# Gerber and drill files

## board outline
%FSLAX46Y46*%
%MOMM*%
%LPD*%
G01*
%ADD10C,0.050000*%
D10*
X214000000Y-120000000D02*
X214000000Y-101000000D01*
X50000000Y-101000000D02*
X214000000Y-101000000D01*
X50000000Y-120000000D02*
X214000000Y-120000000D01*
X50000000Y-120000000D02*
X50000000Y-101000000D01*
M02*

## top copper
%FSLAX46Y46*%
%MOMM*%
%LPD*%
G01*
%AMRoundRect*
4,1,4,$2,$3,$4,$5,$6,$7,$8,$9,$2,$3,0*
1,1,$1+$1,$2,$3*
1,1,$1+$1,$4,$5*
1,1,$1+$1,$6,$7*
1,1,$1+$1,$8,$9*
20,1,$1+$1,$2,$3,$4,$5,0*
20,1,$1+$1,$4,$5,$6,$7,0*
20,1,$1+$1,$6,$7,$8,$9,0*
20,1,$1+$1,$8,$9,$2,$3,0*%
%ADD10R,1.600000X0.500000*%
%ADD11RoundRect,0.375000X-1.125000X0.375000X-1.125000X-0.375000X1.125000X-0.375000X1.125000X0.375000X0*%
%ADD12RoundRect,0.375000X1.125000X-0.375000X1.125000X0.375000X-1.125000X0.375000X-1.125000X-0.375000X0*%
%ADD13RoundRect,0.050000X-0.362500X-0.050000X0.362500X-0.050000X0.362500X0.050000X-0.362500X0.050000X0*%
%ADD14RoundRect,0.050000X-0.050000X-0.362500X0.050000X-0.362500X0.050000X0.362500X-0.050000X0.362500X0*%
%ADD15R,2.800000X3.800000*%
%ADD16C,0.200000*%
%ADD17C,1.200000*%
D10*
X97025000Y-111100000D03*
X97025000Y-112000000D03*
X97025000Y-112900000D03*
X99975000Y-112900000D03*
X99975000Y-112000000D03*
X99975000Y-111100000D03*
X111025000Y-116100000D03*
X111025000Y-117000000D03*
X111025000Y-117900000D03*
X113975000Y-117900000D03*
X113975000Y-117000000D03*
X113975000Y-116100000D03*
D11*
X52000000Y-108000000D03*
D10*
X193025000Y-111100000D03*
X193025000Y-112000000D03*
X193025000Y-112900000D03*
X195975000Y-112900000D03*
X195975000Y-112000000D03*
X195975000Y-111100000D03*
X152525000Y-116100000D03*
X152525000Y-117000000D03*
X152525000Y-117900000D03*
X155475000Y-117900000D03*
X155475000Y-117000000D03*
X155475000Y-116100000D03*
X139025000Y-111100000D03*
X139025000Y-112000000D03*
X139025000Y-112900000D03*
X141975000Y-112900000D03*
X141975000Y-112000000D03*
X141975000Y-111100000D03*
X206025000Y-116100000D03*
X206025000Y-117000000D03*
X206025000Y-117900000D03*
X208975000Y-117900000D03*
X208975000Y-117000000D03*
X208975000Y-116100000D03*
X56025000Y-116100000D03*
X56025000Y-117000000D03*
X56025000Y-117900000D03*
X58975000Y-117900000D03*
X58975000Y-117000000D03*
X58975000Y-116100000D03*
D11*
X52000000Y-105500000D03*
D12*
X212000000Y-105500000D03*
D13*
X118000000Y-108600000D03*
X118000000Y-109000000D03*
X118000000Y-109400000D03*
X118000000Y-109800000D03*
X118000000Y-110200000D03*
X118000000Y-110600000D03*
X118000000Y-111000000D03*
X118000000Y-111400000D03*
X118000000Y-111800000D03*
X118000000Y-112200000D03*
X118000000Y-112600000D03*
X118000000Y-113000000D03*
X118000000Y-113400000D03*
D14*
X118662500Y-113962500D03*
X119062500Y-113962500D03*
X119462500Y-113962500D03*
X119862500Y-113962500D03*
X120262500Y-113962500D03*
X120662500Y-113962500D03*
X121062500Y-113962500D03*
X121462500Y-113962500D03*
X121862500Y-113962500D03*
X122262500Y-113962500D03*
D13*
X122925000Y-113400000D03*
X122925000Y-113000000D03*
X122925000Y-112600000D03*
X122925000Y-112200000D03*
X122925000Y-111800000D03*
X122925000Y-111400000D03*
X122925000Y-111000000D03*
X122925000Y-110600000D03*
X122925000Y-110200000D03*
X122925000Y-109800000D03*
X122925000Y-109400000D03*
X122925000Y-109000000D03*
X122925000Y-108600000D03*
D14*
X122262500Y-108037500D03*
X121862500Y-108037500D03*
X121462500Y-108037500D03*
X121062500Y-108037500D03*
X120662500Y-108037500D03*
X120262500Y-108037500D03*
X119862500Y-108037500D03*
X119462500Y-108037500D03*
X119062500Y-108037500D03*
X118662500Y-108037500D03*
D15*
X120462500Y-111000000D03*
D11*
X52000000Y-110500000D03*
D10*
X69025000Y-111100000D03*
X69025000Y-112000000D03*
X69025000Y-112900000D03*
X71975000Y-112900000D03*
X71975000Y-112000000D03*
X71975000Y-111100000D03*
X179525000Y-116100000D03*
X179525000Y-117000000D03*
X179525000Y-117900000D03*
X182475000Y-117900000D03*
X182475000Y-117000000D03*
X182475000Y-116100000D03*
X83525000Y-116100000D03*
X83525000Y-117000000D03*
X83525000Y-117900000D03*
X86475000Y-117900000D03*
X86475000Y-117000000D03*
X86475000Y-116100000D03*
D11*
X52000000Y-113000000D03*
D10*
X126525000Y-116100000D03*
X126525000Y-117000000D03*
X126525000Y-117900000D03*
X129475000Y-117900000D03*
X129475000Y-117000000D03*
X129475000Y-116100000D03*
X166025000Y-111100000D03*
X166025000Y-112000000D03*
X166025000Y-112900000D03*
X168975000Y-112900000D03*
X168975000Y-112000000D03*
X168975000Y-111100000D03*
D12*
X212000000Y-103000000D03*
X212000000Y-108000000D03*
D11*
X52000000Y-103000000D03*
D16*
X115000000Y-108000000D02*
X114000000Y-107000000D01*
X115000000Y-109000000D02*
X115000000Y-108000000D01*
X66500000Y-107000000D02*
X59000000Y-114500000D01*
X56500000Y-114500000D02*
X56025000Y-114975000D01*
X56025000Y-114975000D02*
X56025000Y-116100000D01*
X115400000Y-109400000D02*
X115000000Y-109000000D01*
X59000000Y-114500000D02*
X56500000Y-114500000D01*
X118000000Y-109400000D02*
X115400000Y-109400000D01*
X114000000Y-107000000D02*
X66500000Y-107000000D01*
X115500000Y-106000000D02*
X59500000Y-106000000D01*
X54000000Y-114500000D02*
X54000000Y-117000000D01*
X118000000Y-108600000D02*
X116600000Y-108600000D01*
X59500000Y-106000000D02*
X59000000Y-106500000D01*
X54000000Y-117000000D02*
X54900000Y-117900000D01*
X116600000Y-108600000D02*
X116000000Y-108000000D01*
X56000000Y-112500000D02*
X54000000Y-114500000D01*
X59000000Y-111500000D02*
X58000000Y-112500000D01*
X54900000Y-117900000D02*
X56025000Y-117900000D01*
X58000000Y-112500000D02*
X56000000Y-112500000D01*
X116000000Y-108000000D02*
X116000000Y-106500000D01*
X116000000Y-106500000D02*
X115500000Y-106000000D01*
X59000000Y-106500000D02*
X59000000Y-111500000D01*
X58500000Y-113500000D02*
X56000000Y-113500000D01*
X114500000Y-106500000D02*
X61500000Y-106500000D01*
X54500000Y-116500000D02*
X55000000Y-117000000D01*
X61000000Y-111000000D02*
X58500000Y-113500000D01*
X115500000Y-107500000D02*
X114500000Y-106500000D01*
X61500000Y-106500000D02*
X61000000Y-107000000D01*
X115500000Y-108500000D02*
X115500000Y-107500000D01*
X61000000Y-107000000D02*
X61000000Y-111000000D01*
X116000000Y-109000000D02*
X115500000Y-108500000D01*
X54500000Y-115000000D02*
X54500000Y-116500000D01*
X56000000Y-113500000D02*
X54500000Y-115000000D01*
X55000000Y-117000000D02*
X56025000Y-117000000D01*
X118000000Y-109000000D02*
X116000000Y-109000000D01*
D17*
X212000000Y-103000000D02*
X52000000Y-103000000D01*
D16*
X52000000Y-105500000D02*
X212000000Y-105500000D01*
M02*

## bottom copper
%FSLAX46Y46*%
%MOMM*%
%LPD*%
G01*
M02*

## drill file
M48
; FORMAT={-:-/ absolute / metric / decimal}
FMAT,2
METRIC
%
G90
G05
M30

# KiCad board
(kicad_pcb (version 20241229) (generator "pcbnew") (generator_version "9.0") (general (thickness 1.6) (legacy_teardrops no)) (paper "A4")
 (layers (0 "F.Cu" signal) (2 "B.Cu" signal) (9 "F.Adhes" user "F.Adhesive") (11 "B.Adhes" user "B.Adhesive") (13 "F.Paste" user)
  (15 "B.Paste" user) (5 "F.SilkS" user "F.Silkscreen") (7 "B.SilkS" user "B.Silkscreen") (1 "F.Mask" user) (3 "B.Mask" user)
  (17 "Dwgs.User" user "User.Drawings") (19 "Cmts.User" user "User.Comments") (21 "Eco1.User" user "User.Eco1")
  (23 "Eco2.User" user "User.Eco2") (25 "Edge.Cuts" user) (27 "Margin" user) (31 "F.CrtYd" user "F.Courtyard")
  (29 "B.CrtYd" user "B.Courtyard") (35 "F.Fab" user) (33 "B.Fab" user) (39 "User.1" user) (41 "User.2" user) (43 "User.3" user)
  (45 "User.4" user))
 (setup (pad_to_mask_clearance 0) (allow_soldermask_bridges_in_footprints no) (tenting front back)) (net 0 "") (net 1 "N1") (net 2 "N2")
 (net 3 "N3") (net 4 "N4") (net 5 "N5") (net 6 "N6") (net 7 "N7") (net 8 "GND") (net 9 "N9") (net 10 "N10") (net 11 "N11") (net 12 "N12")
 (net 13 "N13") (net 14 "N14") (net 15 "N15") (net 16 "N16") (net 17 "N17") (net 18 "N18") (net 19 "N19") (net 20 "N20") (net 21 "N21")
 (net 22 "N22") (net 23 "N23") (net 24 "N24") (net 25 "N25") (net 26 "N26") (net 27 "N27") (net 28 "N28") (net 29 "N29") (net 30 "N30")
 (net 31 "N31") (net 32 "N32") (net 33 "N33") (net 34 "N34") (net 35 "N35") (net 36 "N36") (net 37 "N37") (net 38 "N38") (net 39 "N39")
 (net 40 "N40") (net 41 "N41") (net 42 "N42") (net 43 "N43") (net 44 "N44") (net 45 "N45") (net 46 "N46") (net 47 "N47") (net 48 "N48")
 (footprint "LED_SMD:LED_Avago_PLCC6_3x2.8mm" (layer "F.Cu") (at 98.5 112)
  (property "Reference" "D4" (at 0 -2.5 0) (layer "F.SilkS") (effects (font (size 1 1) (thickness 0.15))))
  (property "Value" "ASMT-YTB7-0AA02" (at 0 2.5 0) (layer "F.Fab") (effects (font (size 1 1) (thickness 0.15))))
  (pad "1" smd rect (at -1.475 -0.9) (size 1.6 0.5) (layers "F.Cu" "F.Mask" "F.Paste") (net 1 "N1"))
  (pad "2" smd rect (at -1.475 0) (size 1.6 0.5) (layers "F.Cu" "F.Mask" "F.Paste") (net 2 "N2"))
  (pad "3" smd rect (at -1.475 0.9) (size 1.6 0.5) (layers "F.Cu" "F.Mask" "F.Paste") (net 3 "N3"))
  (pad "4" smd rect (at 1.475 0.9) (size 1.6 0.5) (layers "F.Cu" "F.Mask" "F.Paste") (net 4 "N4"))
  (pad "5" smd rect (at 1.475 0) (size 1.6 0.5) (layers "F.Cu" "F.Mask" "F.Paste") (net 4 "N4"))
  (pad "6" smd rect (at 1.475 -0.9) (size 1.6 0.5) (layers "F.Cu" "F.Mask" "F.Paste") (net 4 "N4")))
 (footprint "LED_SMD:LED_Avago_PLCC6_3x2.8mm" (layer "F.Cu") (at 112.5 117)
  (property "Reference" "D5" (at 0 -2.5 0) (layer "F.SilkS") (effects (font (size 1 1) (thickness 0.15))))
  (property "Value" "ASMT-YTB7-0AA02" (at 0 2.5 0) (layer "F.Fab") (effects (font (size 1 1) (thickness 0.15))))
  (pad "1" smd rect (at -1.475 -0.9) (size 1.6 0.5) (layers "F.Cu" "F.Mask" "F.Paste") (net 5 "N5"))
  (pad "2" smd rect (at -1.475 0) (size 1.6 0.5) (layers "F.Cu" "F.Mask" "F.Paste") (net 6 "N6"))
  (pad "3" smd rect (at -1.475 0.9) (size 1.6 0.5) (layers "F.Cu" "F.Mask" "F.Paste") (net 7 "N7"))
  (pad "4" smd rect (at 1.475 0.9) (size 1.6 0.5) (layers "F.Cu" "F.Mask" "F.Paste") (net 4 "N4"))
  (pad "5" smd rect (at 1.475 0) (size 1.6 0.5) (layers "F.Cu" "F.Mask" "F.Paste") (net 4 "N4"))
  (pad "6" smd rect (at 1.475 -0.9) (size 1.6 0.5) (layers "F.Cu" "F.Mask" "F.Paste") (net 4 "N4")))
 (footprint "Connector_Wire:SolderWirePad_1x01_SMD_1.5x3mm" (layer "F.Cu") (at 52 108 -90)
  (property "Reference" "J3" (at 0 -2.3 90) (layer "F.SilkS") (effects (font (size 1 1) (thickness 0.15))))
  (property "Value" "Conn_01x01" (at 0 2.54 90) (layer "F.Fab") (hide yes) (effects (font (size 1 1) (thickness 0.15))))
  (pad "1" smd roundrect (at 0 0 270) (size 1.5 3) (layers "F.Cu" "F.Mask") (roundrect_rratio 0.25) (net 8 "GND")))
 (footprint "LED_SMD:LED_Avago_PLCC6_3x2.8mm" (layer "F.Cu") (at 194.5 112)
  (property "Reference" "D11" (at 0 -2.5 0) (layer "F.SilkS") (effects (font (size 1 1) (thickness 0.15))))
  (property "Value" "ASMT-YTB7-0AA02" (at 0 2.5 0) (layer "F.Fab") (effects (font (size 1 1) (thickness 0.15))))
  (pad "1" smd rect (at -1.475 -0.9) (size 1.6 0.5) (layers "F.Cu" "F.Mask" "F.Paste") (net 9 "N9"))
  (pad "2" smd rect (at -1.475 0) (size 1.6 0.5) (layers "F.Cu" "F.Mask" "F.Paste") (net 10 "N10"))
  (pad "3" smd rect (at -1.475 0.9) (size 1.6 0.5) (layers "F.Cu" "F.Mask" "F.Paste") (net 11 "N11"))
  (pad "4" smd rect (at 1.475 0.9) (size 1.6 0.5) (layers "F.Cu" "F.Mask" "F.Paste") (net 4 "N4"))
  (pad "5" smd rect (at 1.475 0) (size 1.6 0.5) (layers "F.Cu" "F.Mask" "F.Paste") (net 4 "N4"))
  (pad "6" smd rect (at 1.475 -0.9) (size 1.6 0.5) (layers "F.Cu" "F.Mask" "F.Paste") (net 4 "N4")))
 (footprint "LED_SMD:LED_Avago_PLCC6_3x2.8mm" (layer "F.Cu") (at 154 117)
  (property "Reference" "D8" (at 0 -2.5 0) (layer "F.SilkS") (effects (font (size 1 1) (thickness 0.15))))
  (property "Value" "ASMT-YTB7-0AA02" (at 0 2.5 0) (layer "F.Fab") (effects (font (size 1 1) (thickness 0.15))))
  (pad "1" smd rect (at -1.475 -0.9) (size 1.6 0.5) (layers "F.Cu" "F.Mask" "F.Paste") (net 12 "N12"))
  (pad "2" smd rect (at -1.475 0) (size 1.6 0.5) (layers "F.Cu" "F.Mask" "F.Paste") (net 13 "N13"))
  (pad "3" smd rect (at -1.475 0.9) (size 1.6 0.5) (layers "F.Cu" "F.Mask" "F.Paste") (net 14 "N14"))
  (pad "4" smd rect (at 1.475 0.9) (size 1.6 0.5) (layers "F.Cu" "F.Mask" "F.Paste") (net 4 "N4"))
  (pad "5" smd rect (at 1.475 0) (size 1.6 0.5) (layers "F.Cu" "F.Mask" "F.Paste") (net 4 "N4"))
  (pad "6" smd rect (at 1.475 -0.9) (size 1.6 0.5) (layers "F.Cu" "F.Mask" "F.Paste") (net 4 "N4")))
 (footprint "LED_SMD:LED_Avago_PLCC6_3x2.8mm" (layer "F.Cu") (at 140.5 112)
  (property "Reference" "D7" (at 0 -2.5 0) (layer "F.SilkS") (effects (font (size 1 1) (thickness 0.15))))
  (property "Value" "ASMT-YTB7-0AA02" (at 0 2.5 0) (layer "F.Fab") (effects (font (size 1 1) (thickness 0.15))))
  (pad "1" smd rect (at -1.475 -0.9) (size 1.6 0.5) (layers "F.Cu" "F.Mask" "F.Paste") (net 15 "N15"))
  (pad "2" smd rect (at -1.475 0) (size 1.6 0.5) (layers "F.Cu" "F.Mask" "F.Paste") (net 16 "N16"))
  (pad "3" smd rect (at -1.475 0.9) (size 1.6 0.5) (layers "F.Cu" "F.Mask" "F.Paste") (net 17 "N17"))
  (pad "4" smd rect (at 1.475 0.9) (size 1.6 0.5) (layers "F.Cu" "F.Mask" "F.Paste") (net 4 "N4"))
  (pad "5" smd rect (at 1.475 0) (size 1.6 0.5) (layers "F.Cu" "F.Mask" "F.Paste") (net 4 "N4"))
  (pad "6" smd rect (at 1.475 -0.9) (size 1.6 0.5) (layers "F.Cu" "F.Mask" "F.Paste") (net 4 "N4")))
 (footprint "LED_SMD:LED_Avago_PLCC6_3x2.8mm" (layer "F.Cu") (at 207.5 117)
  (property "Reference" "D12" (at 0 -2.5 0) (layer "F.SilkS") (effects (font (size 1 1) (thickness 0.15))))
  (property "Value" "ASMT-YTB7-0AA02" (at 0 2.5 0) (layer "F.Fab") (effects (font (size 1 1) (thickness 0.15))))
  (pad "1" smd rect (at -1.475 -0.9) (size 1.6 0.5) (layers "F.Cu" "F.Mask" "F.Paste") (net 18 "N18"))
  (pad "2" smd rect (at -1.475 0) (size 1.6 0.5) (layers "F.Cu" "F.Mask" "F.Paste") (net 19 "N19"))
  (pad "3" smd rect (at -1.475 0.9) (size 1.6 0.5) (layers "F.Cu" "F.Mask" "F.Paste") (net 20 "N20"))
  (pad "4" smd rect (at 1.475 0.9) (size 1.6 0.5) (layers "F.Cu" "F.Mask" "F.Paste") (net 4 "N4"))
  (pad "5" smd rect (at 1.475 0) (size 1.6 0.5) (layers "F.Cu" "F.Mask" "F.Paste") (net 4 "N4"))
  (pad "6" smd rect (at 1.475 -0.9) (size 1.6 0.5) (layers "F.Cu" "F.Mask" "F.Paste") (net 4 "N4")))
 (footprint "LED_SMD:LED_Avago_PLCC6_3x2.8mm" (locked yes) (layer "F.Cu") (at 57.5 117)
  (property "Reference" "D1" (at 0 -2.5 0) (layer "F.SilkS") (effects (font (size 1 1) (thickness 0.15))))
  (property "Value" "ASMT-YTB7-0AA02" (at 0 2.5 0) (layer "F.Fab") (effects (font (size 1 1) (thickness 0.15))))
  (pad "1" smd rect (at -1.475 -0.9) (size 1.6 0.5) (layers "F.Cu" "F.Mask" "F.Paste") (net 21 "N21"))
  (pad "2" smd rect (at -1.475 0) (size 1.6 0.5) (layers "F.Cu" "F.Mask" "F.Paste") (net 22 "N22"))
  (pad "3" smd rect (at -1.475 0.9) (size 1.6 0.5) (layers "F.Cu" "F.Mask" "F.Paste") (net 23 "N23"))
  (pad "4" smd rect (at 1.475 0.9) (size 1.6 0.5) (layers "F.Cu" "F.Mask" "F.Paste") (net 4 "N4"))
  (pad "5" smd rect (at 1.475 0) (size 1.6 0.5) (layers "F.Cu" "F.Mask" "F.Paste") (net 4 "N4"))
  (pad "6" smd rect (at 1.475 -0.9) (size 1.6 0.5) (layers "F.Cu" "F.Mask" "F.Paste") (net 4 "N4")))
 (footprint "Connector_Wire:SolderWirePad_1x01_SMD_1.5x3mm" (layer "F.Cu") (at 52 105.5 -90)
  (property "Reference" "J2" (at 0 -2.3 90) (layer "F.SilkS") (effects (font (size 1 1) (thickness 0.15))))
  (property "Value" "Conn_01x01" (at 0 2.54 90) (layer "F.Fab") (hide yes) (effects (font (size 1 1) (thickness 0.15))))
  (pad "1" smd roundrect (at 0 0 270) (size 1.5 3) (layers "F.Cu" "F.Mask") (roundrect_rratio 0.25) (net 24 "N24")))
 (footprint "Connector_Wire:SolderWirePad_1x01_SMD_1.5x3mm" (layer "F.Cu") (at 212 105.5 90)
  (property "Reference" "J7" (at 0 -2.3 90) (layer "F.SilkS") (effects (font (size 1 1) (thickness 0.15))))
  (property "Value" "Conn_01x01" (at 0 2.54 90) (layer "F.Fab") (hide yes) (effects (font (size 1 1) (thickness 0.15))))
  (pad "1" smd roundrect (at 0 0 90) (size 1.5 3) (layers "F.Cu" "F.Mask") (roundrect_rratio 0.25) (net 24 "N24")))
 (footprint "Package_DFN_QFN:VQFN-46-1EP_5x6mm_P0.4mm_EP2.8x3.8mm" (layer "F.Cu") (at 120.4625 111)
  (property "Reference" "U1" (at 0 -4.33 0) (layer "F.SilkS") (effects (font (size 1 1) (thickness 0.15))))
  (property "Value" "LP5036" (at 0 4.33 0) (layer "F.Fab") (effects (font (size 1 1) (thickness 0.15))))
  (pad "" smd roundrect (at -0.7 -1.27) (size 1.13 1.02) (layers "F.Paste") (roundrect_rratio 0.245098))
  (pad "" smd roundrect (at -0.7 0) (size 1.13 1.02) (layers "F.Paste") (roundrect_rratio 0.245098))
  (pad "" smd roundrect (at -0.7 1.27) (size 1.13 1.02) (layers "F.Paste") (roundrect_rratio 0.245098))
  (pad "" smd roundrect (at 0.7 -1.27) (size 1.13 1.02) (layers "F.Paste") (roundrect_rratio 0.245098))
  (pad "" smd roundrect (at 0.7 0) (size 1.13 1.02) (layers "F.Paste") (roundrect_rratio 0.245098))
  (pad "" smd roundrect (at 0.7 1.27) (size 1.13 1.02) (layers "F.Paste") (roundrect_rratio 0.245098))
  (pad "1" smd roundrect (at -2.4625 -2.4) (size 0.825 0.2) (layers "F.Cu" "F.Mask" "F.Paste") (roundrect_rratio 0.25) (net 23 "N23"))
  (pad "2" smd roundrect (at -2.4625 -2) (size 0.825 0.2) (layers "F.Cu" "F.Mask" "F.Paste") (roundrect_rratio 0.25) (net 22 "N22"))
  (pad "3" smd roundrect (at -2.4625 -1.6) (size 0.825 0.2) (layers "F.Cu" "F.Mask" "F.Paste") (roundrect_rratio 0.25) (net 21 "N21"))
  (pad "4" smd roundrect (at -2.4625 -1.2) (size 0.825 0.2) (layers "F.Cu" "F.Mask" "F.Paste") (roundrect_rratio 0.25) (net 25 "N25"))
  (pad "5" smd roundrect (at -2.4625 -0.8) (size 0.825 0.2) (layers "F.Cu" "F.Mask" "F.Paste") (roundrect_rratio 0.25) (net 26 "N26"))
  (pad "6" smd roundrect (at -2.4625 -0.4) (size 0.825 0.2) (layers "F.Cu" "F.Mask" "F.Paste") (roundrect_rratio 0.25) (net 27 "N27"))
  (pad "7" smd roundrect (at -2.4625 0) (size 0.825 0.2) (layers "F.Cu" "F.Mask" "F.Paste") (roundrect_rratio 0.25) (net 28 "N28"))
  (pad "8" smd roundrect (at -2.4625 0.4) (size 0.825 0.2) (layers "F.Cu" "F.Mask" "F.Paste") (roundrect_rratio 0.25) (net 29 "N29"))
  (pad "9" smd roundrect (at -2.4625 0.8) (size 0.825 0.2) (layers "F.Cu" "F.Mask" "F.Paste") (roundrect_rratio 0.25) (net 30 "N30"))
  (pad "10" smd roundrect (at -2.4625 1.2) (size 0.825 0.2) (layers "F.Cu" "F.Mask" "F.Paste") (roundrect_rratio 0.25) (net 3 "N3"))
  (pad "11" smd roundrect (at -2.4625 1.6) (size 0.825 0.2) (layers "F.Cu" "F.Mask" "F.Paste") (roundrect_rratio 0.25) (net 2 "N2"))
  (pad "12" smd roundrect (at -2.4625 2) (size 0.825 0.2) (layers "F.Cu" "F.Mask" "F.Paste") (roundrect_rratio 0.25) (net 1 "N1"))
  (pad "13" smd roundrect (at -2.4625 2.4) (size 0.825 0.2) (layers "F.Cu" "F.Mask" "F.Paste") (roundrect_rratio 0.25) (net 7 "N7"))
  (pad "14" smd roundrect (at -1.8 2.9625) (size 0.2 0.825) (layers "F.Cu" "F.Mask" "F.Paste") (roundrect_rratio 0.25) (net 6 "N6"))
  (pad "15" smd roundrect (at -1.4 2.9625) (size 0.2 0.825) (layers "F.Cu" "F.Mask" "F.Paste") (roundrect_rratio 0.25) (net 5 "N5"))
  (pad "16" smd roundrect (at -1 2.9625) (size 0.2 0.825) (layers "F.Cu" "F.Mask" "F.Paste") (roundrect_rratio 0.25) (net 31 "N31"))
  (pad "17" smd roundrect (at -0.6 2.9625) (size 0.2 0.825) (layers "F.Cu" "F.Mask" "F.Paste") (roundrect_rratio 0.25) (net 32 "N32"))
  (pad "18" smd roundrect (at -0.2 2.9625) (size 0.2 0.825) (layers "F.Cu" "F.Mask" "F.Paste") (roundrect_rratio 0.25) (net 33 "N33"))
  (pad "19" smd roundrect (at 0.2 2.9625) (size 0.2 0.825) (layers "F.Cu" "F.Mask" "F.Paste") (roundrect_rratio 0.25) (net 17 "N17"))
  (pad "20" smd roundrect (at 0.6 2.9625) (size 0.2 0.825) (layers "F.Cu" "F.Mask" "F.Paste") (roundrect_rratio 0.25) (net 16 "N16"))
  (pad "21" smd roundrect (at 1 2.9625) (size 0.2 0.825) (layers "F.Cu" "F.Mask" "F.Paste") (roundrect_rratio 0.25) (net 15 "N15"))
  (pad "22" smd roundrect (at 1.4 2.9625) (size 0.2 0.825) (layers "F.Cu" "F.Mask" "F.Paste") (roundrect_rratio 0.25) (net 14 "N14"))
  (pad "23" smd roundrect (at 1.8 2.9625) (size 0.2 0.825) (layers "F.Cu" "F.Mask" "F.Paste") (roundrect_rratio 0.25) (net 13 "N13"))
  (pad "24" smd roundrect (at 2.4625 2.4) (size 0.825 0.2) (layers "F.Cu" "F.Mask" "F.Paste") (roundrect_rratio 0.25) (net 12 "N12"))
  (pad "25" smd roundrect (at 2.4625 2) (size 0.825 0.2) (layers "F.Cu" "F.Mask" "F.Paste") (roundrect_rratio 0.25) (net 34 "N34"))
  (pad "26" smd roundrect (at 2.4625 1.6) (size 0.825 0.2) (layers "F.Cu" "F.Mask" "F.Paste") (roundrect_rratio 0.25) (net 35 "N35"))
  (pad "27" smd roundrect (at 2.4625 1.2) (size 0.825 0.2) (layers "F.Cu" "F.Mask" "F.Paste") (roundrect_rratio 0.25) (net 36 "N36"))
  (pad "28" smd roundrect (at 2.4625 0.8) (size 0.825 0.2) (layers "F.Cu" "F.Mask" "F.Paste") (roundrect_rratio 0.25) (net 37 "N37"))
  (pad "29" smd roundrect (at 2.4625 0.4) (size 0.825 0.2) (layers "F.Cu" "F.Mask" "F.Paste") (roundrect_rratio 0.25) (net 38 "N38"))
  (pad "30" smd roundrect (at 2.4625 0) (size 0.825 0.2) (layers "F.Cu" "F.Mask" "F.Paste") (roundrect_rratio 0.25) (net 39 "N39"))
  (pad "31" smd roundrect (at 2.4625 -0.4) (size 0.825 0.2) (layers "F.Cu" "F.Mask" "F.Paste") (roundrect_rratio 0.25) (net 11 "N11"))
  (pad "32" smd roundrect (at 2.4625 -0.8) (size 0.825 0.2) (layers "F.Cu" "F.Mask" "F.Paste") (roundrect_rratio 0.25) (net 10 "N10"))
  (pad "33" smd roundrect (at 2.4625 -1.2) (size 0.825 0.2) (layers "F.Cu" "F.Mask" "F.Paste") (roundrect_rratio 0.25) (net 9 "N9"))
  (pad "34" smd roundrect (at 2.4625 -1.6) (size 0.825 0.2) (layers "F.Cu" "F.Mask" "F.Paste") (roundrect_rratio 0.25) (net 20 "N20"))
  (pad "35" smd roundrect (at 2.4625 -2) (size 0.825 0.2) (layers "F.Cu" "F.Mask" "F.Paste") (roundrect_rratio 0.25) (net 19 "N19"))
  (pad "36" smd roundrect (at 2.4625 -2.4) (size 0.825 0.2) (layers "F.Cu" "F.Mask" "F.Paste") (roundrect_rratio 0.25) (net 18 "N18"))
  (pad "37" smd roundrect (at 1.8 -2.9625) (size 0.2 0.825) (layers "F.Cu" "F.Mask" "F.Paste") (roundrect_rratio 0.25) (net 8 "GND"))
  (pad "38" smd roundrect (at 1.4 -2.9625) (size 0.2 0.825) (layers "F.Cu" "F.Mask" "F.Paste") (roundrect_rratio 0.25) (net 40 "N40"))
  (pad "39" smd roundrect (at 1 -2.9625) (size 0.2 0.825) (layers "F.Cu" "F.Mask" "F.Paste") (roundrect_rratio 0.25) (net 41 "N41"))
  (pad "40" smd roundrect (at 0.6 -2.9625) (size 0.2 0.825) (layers "F.Cu" "F.Mask" "F.Paste") (roundrect_rratio 0.25) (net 24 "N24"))
  (pad "41" smd roundrect (at 0.2 -2.9625) (size 0.2 0.825) (layers "F.Cu" "F.Mask" "F.Paste") (roundrect_rratio 0.25) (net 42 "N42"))
  (pad "42" smd roundrect (at -0.2 -2.9625) (size 0.2 0.825) (layers "F.Cu" "F.Mask" "F.Paste") (roundrect_rratio 0.25) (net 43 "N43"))
  (pad "43" smd roundrect (at -0.6 -2.9625) (size 0.2 0.825) (layers "F.Cu" "F.Mask" "F.Paste") (roundrect_rratio 0.25) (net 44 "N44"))
  (pad "44" smd roundrect (at -1 -2.9625) (size 0.2 0.825) (layers "F.Cu" "F.Mask" "F.Paste") (roundrect_rratio 0.25) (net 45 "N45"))
  (pad "45" smd roundrect (at -1.4 -2.9625) (size 0.2 0.825) (layers "F.Cu" "F.Mask" "F.Paste") (roundrect_rratio 0.25) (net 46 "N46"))
  (pad "46" smd roundrect (at -1.8 -2.9625) (size 0.2 0.825) (layers "F.Cu" "F.Mask" "F.Paste") (roundrect_rratio 0.25) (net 8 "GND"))
  (pad "47" smd rect (at 0 0) (size 2.8 3.8) (layers "F.Cu" "F.Mask") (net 8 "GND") (zone_connect 2)))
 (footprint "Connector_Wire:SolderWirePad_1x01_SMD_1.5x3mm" (layer "F.Cu") (at 52 110.5 -90)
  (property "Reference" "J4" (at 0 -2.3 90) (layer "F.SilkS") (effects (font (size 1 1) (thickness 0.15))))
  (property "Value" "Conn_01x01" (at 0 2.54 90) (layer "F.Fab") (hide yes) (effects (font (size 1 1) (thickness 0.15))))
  (pad "1" smd roundrect (at 0 0 270) (size 1.5 3) (layers "F.Cu" "F.Mask") (roundrect_rratio 0.25) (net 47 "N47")))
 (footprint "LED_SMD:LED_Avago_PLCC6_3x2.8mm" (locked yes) (layer "F.Cu") (at 70.5 112)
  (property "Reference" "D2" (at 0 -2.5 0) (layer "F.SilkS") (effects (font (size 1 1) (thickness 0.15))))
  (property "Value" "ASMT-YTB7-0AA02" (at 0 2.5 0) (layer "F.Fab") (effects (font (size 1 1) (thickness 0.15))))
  (pad "1" smd rect (at -1.475 -0.9) (size 1.6 0.5) (layers "F.Cu" "F.Mask" "F.Paste") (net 27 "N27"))
  (pad "2" smd rect (at -1.475 0) (size 1.6 0.5) (layers "F.Cu" "F.Mask" "F.Paste") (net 26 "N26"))
  (pad "3" smd rect (at -1.475 0.9) (size 1.6 0.5) (layers "F.Cu" "F.Mask" "F.Paste") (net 25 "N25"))
  (pad "4" smd rect (at 1.475 0.9) (size 1.6 0.5) (layers "F.Cu" "F.Mask" "F.Paste") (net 4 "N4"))
  (pad "5" smd rect (at 1.475 0) (size 1.6 0.5) (layers "F.Cu" "F.Mask" "F.Paste") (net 4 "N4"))
  (pad "6" smd rect (at 1.475 -0.9) (size 1.6 0.5) (layers "F.Cu" "F.Mask" "F.Paste") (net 4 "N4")))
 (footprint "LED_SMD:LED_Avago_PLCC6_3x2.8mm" (layer "F.Cu") (at 181 117)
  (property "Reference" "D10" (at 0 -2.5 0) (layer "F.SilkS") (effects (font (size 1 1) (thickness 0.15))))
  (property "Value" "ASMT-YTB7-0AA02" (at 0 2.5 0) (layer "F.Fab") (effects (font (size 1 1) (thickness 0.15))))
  (pad "1" smd rect (at -1.475 -0.9) (size 1.6 0.5) (layers "F.Cu" "F.Mask" "F.Paste") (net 39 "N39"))
  (pad "2" smd rect (at -1.475 0) (size 1.6 0.5) (layers "F.Cu" "F.Mask" "F.Paste") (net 38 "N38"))
  (pad "3" smd rect (at -1.475 0.9) (size 1.6 0.5) (layers "F.Cu" "F.Mask" "F.Paste") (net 37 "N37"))
  (pad "4" smd rect (at 1.475 0.9) (size 1.6 0.5) (layers "F.Cu" "F.Mask" "F.Paste") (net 4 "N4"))
  (pad "5" smd rect (at 1.475 0) (size 1.6 0.5) (layers "F.Cu" "F.Mask" "F.Paste") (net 4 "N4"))
  (pad "6" smd rect (at 1.475 -0.9) (size 1.6 0.5) (layers "F.Cu" "F.Mask" "F.Paste") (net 4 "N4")))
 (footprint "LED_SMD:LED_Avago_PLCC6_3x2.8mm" (layer "F.Cu") (at 85 117)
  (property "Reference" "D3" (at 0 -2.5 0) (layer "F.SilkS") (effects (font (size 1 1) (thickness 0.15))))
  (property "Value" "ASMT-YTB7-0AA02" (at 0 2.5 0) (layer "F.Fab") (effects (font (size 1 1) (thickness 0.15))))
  (pad "1" smd rect (at -1.475 -0.9) (size 1.6 0.5) (layers "F.Cu" "F.Mask" "F.Paste") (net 30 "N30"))
  (pad "2" smd rect (at -1.475 0) (size 1.6 0.5) (layers "F.Cu" "F.Mask" "F.Paste") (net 29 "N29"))
  (pad "3" smd rect (at -1.475 0.9) (size 1.6 0.5) (layers "F.Cu" "F.Mask" "F.Paste") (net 28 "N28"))
  (pad "4" smd rect (at 1.475 0.9) (size 1.6 0.5) (layers "F.Cu" "F.Mask" "F.Paste") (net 4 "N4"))
  (pad "5" smd rect (at 1.475 0) (size 1.6 0.5) (layers "F.Cu" "F.Mask" "F.Paste") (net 4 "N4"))
  (pad "6" smd rect (at 1.475 -0.9) (size 1.6 0.5) (layers "F.Cu" "F.Mask" "F.Paste") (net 4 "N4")))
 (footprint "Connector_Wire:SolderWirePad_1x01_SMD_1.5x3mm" (layer "F.Cu") (at 52 113 -90)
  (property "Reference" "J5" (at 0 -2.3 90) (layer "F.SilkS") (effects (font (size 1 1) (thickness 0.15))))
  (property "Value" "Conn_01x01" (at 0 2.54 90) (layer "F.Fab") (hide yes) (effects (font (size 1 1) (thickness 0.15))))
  (pad "1" smd roundrect (at 0 0 270) (size 1.5 3) (layers "F.Cu" "F.Mask") (roundrect_rratio 0.25) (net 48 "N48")))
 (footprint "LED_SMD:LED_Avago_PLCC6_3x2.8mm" (layer "F.Cu") (at 128 117)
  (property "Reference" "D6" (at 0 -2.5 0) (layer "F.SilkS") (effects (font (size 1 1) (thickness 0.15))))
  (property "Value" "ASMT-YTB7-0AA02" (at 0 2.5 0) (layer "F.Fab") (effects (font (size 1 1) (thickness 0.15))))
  (pad "1" smd rect (at -1.475 -0.9) (size 1.6 0.5) (layers "F.Cu" "F.Mask" "F.Paste") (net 33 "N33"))
  (pad "2" smd rect (at -1.475 0) (size 1.6 0.5) (layers "F.Cu" "F.Mask" "F.Paste") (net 32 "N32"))
  (pad "3" smd rect (at -1.475 0.9) (size 1.6 0.5) (layers "F.Cu" "F.Mask" "F.Paste") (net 31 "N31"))
  (pad "4" smd rect (at 1.475 0.9) (size 1.6 0.5) (layers "F.Cu" "F.Mask" "F.Paste") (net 4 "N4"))
  (pad "5" smd rect (at 1.475 0) (size 1.6 0.5) (layers "F.Cu" "F.Mask" "F.Paste") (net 4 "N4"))
  (pad "6" smd rect (at 1.475 -0.9) (size 1.6 0.5) (layers "F.Cu" "F.Mask" "F.Paste") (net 4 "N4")))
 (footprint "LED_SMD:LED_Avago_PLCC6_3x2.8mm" (layer "F.Cu") (at 167.5 112)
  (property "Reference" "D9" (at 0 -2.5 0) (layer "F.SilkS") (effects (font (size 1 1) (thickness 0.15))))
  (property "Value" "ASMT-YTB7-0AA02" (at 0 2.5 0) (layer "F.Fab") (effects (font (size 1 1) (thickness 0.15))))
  (pad "1" smd rect (at -1.475 -0.9) (size 1.6 0.5) (layers "F.Cu" "F.Mask" "F.Paste") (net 36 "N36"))
  (pad "2" smd rect (at -1.475 0) (size 1.6 0.5) (layers "F.Cu" "F.Mask" "F.Paste") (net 35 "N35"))
  (pad "3" smd rect (at -1.475 0.9) (size 1.6 0.5) (layers "F.Cu" "F.Mask" "F.Paste") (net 34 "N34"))
  (pad "4" smd rect (at 1.475 0.9) (size 1.6 0.5) (layers "F.Cu" "F.Mask" "F.Paste") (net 4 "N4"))
  (pad "5" smd rect (at 1.475 0) (size 1.6 0.5) (layers "F.Cu" "F.Mask" "F.Paste") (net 4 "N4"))
  (pad "6" smd rect (at 1.475 -0.9) (size 1.6 0.5) (layers "F.Cu" "F.Mask" "F.Paste") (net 4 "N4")))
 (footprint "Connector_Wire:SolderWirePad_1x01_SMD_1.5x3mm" (layer "F.Cu") (at 212 103 90)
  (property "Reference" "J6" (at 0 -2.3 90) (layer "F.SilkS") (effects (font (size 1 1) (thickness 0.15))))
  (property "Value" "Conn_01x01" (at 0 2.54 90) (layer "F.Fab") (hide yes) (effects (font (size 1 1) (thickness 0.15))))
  (pad "1" smd roundrect (at 0 0 90) (size 1.5 3) (layers "F.Cu" "F.Mask") (roundrect_rratio 0.25) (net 4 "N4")))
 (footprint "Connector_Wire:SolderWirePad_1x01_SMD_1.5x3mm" (layer "F.Cu") (at 212 108 90)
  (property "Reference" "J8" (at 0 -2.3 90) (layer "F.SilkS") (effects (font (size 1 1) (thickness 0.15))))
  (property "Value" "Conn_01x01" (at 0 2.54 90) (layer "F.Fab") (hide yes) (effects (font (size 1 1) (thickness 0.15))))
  (pad "1" smd roundrect (at 0 0 90) (size 1.5 3) (layers "F.Cu" "F.Mask") (roundrect_rratio 0.25) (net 8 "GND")))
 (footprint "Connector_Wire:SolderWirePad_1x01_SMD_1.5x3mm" (layer "F.Cu") (at 52 103 -90)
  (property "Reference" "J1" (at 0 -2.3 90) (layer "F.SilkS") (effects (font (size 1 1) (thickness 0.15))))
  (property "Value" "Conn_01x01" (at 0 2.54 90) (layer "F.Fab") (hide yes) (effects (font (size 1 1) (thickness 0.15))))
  (pad "1" smd roundrect (at 0 0 270) (size 1.5 3) (layers "F.Cu" "F.Mask") (roundrect_rratio 0.25) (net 4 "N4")))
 (gr_line (start 214 120) (end 214 101) (stroke (width 0.05) (type default)) (layer "Edge.Cuts"))
 (gr_line (start 50 101) (end 214 101) (stroke (width 0.05) (type solid)) (layer "Edge.Cuts"))
 (gr_line (start 50 120) (end 214 120) (stroke (width 0.05) (type solid)) (layer "Edge.Cuts"))
 (gr_line (start 50 120) (end 50 101) (stroke (width 0.05) (type default)) (layer "Edge.Cuts"))
 (segment (start 115 108) (end 114 107) (width 0.2) (layer "F.Cu") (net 21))
 (segment (start 115 109) (end 115 108) (width 0.2) (layer "F.Cu") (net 21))
 (segment (start 66.5 107) (end 59 114.5) (width 0.2) (layer "F.Cu") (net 21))
 (segment (start 56.5 114.5) (end 56.025 114.975) (width 0.2) (layer "F.Cu") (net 21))
 (segment (start 56.025 114.975) (end 56.025 116.1) (width 0.2) (layer "F.Cu") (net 21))
 (segment (start 115.4 109.4) (end 115 109) (width 0.2) (layer "F.Cu") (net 21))
 (segment (start 59 114.5) (end 56.5 114.5) (width 0.2) (layer "F.Cu") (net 21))
 (segment (start 118 109.4) (end 115.4 109.4) (width 0.2) (layer "F.Cu") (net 21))
 (segment (start 114 107) (end 66.5 107) (width 0.2) (layer "F.Cu") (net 21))
 (segment (start 115.5 106) (end 59.5 106) (width 0.2) (layer "F.Cu") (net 23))
 (segment (start 54 114.5) (end 54 117) (width 0.2) (layer "F.Cu") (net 23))
 (segment (start 118 108.6) (end 116.6 108.6) (width 0.2) (layer "F.Cu") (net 23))
 (segment (start 59.5 106) (end 59 106.5) (width 0.2) (layer "F.Cu") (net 23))
 (segment (start 54 117) (end 54.9 117.9) (width 0.2) (layer "F.Cu") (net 23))
 (segment (start 116.6 108.6) (end 116 108) (width 0.2) (layer "F.Cu") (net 23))
 (segment (start 56 112.5) (end 54 114.5) (width 0.2) (layer "F.Cu") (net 23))
 (segment (start 59 111.5) (end 58 112.5) (width 0.2) (layer "F.Cu") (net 23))
 (segment (start 54.9 117.9) (end 56.025 117.9) (width 0.2) (layer "F.Cu") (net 23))
 (segment (start 58 112.5) (end 56 112.5) (width 0.2) (layer "F.Cu") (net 23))
 (segment (start 116 108) (end 116 106.5) (width 0.2) (layer "F.Cu") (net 23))
 (segment (start 116 106.5) (end 115.5 106) (width 0.2) (layer "F.Cu") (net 23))
 (segment (start 59 106.5) (end 59 111.5) (width 0.2) (layer "F.Cu") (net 23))
 (segment (start 58.5 113.5) (end 56 113.5) (width 0.2) (layer "F.Cu") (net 22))
 (segment (start 114.5 106.5) (end 61.5 106.5) (width 0.2) (layer "F.Cu") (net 22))
 (segment (start 54.5 116.5) (end 55 117) (width 0.2) (layer "F.Cu") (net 22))
 (segment (start 61 111) (end 58.5 113.5) (width 0.2) (layer "F.Cu") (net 22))
 (segment (start 115.5 107.5) (end 114.5 106.5) (width 0.2) (layer "F.Cu") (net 22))
 (segment (start 61.5 106.5) (end 61 107) (width 0.2) (layer "F.Cu") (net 22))
 (segment (start 115.5 108.5) (end 115.5 107.5) (width 0.2) (layer "F.Cu") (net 22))
 (segment (start 61 107) (end 61 111) (width 0.2) (layer "F.Cu") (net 22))
 (segment (start 116 109) (end 115.5 108.5) (width 0.2) (layer "F.Cu") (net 22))
 (segment (start 54.5 115) (end 54.5 116.5) (width 0.2) (layer "F.Cu") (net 22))
 (segment (start 56 113.5) (end 54.5 115) (width 0.2) (layer "F.Cu") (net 22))
 (segment (start 55 117) (end 56.025 117) (width 0.2) (layer "F.Cu") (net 22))
 (segment (start 118 109) (end 116 109) (width 0.2) (layer "F.Cu") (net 22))
 (segment (start 212 103) (end 52 103) (width 1.2) (layer "F.Cu") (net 4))
 (segment (start 52 105.5) (end 212 105.5) (width 0.2) (layer "F.Cu") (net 24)))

